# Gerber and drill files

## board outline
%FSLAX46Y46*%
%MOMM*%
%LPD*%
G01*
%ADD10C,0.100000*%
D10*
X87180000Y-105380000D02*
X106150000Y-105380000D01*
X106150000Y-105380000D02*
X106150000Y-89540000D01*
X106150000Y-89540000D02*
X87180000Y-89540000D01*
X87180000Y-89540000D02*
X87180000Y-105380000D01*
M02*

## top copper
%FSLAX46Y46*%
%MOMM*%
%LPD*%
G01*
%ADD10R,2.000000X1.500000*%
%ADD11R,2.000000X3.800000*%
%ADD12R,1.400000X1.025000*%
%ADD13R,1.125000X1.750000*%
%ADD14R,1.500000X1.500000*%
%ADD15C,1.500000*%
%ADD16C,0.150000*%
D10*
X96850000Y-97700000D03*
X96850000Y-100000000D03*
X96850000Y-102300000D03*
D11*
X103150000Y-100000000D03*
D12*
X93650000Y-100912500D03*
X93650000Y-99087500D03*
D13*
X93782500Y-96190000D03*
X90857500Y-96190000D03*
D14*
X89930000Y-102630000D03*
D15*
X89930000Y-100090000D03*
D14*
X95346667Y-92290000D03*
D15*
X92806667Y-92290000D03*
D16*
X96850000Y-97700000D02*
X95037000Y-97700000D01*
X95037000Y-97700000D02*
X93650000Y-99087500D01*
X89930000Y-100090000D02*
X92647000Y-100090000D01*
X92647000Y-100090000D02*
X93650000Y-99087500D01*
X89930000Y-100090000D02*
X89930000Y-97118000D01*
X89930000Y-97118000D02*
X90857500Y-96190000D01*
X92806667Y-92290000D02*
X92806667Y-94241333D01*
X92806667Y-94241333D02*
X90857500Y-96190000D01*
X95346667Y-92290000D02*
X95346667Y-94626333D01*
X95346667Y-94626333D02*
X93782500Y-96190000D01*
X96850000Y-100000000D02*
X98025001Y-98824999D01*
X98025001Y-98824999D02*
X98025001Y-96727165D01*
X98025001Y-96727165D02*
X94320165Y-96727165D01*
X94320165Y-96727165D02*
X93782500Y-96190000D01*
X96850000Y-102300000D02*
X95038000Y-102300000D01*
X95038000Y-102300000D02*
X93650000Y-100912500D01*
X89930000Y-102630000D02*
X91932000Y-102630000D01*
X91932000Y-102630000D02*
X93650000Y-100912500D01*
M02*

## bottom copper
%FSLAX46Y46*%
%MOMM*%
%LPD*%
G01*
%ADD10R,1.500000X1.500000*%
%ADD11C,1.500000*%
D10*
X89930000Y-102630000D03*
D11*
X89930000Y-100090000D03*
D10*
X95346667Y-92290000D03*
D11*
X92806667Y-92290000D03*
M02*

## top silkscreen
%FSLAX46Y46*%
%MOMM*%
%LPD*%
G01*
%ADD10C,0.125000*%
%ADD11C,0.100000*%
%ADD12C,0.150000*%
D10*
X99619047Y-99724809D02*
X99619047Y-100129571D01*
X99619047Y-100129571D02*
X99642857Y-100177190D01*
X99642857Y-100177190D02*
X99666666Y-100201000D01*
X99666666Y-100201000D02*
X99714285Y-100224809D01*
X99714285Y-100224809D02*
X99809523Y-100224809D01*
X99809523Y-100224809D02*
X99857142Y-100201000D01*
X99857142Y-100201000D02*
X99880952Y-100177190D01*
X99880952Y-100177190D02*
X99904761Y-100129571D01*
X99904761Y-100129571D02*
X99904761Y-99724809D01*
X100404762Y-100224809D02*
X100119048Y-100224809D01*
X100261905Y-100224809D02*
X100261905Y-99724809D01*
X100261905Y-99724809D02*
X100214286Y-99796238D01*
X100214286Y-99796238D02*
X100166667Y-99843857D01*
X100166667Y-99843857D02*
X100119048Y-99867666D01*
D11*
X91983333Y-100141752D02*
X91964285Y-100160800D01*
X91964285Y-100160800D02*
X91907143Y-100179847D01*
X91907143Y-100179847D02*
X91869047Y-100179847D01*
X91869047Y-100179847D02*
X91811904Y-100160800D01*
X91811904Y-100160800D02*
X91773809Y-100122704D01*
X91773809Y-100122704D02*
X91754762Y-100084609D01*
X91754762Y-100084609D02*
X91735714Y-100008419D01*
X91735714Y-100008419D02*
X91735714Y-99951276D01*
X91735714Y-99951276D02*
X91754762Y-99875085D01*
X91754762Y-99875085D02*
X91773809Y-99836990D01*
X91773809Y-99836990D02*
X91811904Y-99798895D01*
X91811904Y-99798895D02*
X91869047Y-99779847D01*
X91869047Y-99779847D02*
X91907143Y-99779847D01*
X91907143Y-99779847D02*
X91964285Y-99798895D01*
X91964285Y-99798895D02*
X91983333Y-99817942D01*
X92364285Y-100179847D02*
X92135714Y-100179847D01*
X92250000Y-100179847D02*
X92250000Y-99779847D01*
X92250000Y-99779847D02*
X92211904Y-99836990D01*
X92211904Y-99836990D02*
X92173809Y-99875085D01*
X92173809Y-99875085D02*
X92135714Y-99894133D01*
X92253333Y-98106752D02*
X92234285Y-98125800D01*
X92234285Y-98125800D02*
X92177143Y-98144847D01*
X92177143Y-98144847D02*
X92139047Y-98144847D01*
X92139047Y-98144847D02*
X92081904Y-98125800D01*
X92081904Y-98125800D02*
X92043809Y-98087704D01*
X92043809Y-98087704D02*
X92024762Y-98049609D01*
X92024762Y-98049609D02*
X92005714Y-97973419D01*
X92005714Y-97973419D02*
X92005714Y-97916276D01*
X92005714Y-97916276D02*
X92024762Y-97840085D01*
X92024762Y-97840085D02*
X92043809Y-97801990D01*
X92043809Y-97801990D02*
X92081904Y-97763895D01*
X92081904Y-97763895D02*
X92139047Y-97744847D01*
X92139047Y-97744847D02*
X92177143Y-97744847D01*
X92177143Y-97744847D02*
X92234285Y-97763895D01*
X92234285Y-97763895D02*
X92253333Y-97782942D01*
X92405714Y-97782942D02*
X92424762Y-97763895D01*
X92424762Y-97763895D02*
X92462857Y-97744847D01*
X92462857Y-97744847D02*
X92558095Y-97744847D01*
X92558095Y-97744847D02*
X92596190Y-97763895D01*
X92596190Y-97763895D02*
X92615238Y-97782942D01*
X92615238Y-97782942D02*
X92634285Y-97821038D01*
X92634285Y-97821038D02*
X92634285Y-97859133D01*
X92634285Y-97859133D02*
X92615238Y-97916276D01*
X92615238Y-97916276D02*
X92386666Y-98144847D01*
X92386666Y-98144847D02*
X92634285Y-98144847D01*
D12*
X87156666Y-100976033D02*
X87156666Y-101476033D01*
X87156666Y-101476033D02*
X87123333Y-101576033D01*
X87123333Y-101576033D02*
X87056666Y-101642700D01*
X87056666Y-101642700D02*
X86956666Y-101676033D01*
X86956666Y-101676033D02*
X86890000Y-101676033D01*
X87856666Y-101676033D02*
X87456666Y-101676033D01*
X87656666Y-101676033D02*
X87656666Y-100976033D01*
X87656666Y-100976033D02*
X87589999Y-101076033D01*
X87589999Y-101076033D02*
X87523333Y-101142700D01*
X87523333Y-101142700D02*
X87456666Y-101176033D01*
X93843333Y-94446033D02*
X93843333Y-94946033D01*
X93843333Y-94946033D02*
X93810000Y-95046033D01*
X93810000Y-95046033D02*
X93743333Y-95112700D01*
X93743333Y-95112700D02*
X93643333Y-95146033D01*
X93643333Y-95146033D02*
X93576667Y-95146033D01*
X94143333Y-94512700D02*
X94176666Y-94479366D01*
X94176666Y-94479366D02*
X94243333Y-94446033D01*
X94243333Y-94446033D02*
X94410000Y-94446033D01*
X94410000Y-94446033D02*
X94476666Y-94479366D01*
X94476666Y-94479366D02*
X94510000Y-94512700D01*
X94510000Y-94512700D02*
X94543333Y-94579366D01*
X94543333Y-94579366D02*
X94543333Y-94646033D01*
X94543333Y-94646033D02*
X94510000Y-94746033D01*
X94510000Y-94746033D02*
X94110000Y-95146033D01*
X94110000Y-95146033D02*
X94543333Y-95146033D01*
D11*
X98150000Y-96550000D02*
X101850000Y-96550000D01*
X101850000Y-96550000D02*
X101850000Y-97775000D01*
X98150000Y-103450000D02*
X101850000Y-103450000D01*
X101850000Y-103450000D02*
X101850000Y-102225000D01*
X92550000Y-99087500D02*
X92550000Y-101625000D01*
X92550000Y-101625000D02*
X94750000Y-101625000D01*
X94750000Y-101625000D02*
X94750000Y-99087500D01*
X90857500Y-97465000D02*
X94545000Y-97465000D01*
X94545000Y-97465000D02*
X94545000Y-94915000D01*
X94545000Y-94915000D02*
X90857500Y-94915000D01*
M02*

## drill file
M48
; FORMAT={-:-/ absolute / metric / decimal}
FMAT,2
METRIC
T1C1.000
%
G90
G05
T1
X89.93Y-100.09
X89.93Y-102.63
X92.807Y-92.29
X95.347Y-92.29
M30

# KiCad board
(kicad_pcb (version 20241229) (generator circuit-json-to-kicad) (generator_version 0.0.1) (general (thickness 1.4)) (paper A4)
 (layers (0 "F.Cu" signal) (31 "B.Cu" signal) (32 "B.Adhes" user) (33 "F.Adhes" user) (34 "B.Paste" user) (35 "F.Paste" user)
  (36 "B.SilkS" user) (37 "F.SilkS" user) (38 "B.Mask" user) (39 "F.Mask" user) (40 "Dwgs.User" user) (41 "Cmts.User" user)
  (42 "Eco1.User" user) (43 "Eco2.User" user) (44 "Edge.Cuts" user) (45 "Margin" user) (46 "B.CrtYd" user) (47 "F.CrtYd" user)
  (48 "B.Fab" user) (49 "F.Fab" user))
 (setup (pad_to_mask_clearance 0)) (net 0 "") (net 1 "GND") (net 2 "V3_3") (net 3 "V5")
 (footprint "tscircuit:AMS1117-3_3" (layer F.Cu) (at 100 100 0)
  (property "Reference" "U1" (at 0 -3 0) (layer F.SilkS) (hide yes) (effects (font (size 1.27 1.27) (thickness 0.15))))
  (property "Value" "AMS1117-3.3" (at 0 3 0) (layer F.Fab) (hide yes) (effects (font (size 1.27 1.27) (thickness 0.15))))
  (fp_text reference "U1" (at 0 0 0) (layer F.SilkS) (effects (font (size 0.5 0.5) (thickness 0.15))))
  (fp_line (start -1.85 -3.45) (end 1.85 -3.45) (stroke (width 0.1) (type default)) (layer F.SilkS))
  (fp_line (start 1.85 -3.45) (end 1.85 -2.225) (stroke (width 0.1) (type default)) (layer F.SilkS))
  (fp_line (start -1.85 3.45) (end 1.85 3.45) (stroke (width 0.1) (type default)) (layer F.SilkS))
  (fp_line (start 1.85 3.45) (end 1.85 2.225) (stroke (width 0.1) (type default)) (layer F.SilkS))
  (pad "1" smd rect (at -3.15 -2.3 0) (size 2 1.5) (layers F.Cu F.Paste F.Mask) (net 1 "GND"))
  (pad "2" smd rect (at -3.15 0 0) (size 2 1.5) (layers F.Cu F.Paste F.Mask) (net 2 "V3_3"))
  (pad "3" smd rect (at -3.15 2.3 0) (size 2 1.5) (layers F.Cu F.Paste F.Mask) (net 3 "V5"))
  (pad "4" smd rect (at 3.15 0 0) (size 2 3.8) (layers F.Cu F.Paste F.Mask)))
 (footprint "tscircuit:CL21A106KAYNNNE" (layer F.Cu) (at 93.65 100 90)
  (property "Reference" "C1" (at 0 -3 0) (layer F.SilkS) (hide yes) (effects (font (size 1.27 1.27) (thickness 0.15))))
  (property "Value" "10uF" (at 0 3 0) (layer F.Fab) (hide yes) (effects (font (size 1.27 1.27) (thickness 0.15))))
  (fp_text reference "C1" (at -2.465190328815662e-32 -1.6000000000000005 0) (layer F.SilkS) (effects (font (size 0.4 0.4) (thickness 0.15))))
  (fp_line (start 0.9125 -1.1000000000000005) (end -1.6249999999999998 -1.1000000000000005) (stroke (width 0.1) (type default))
   (layer F.SilkS))
  (fp_line (start -1.6249999999999998 -1.1000000000000005) (end -1.6249999999999998 1.1000000000000005) (stroke (width 0.1) (type default))
   (layer F.SilkS))
  (fp_line (start -1.6249999999999998 1.1000000000000005) (end 0.9125 1.1000000000000005) (stroke (width 0.1) (type default))
   (layer F.SilkS))
  (pad "1" smd rect (at -0.9125 0 0) (size 1.4 1.025) (layers F.Cu F.Paste F.Mask) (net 3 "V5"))
  (pad "2" smd rect (at 0.9125 0 0) (size 1.4 1.025) (layers F.Cu F.Paste F.Mask) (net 1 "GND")))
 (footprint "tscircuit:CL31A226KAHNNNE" (layer F.Cu) (at 92.32 96.19 180)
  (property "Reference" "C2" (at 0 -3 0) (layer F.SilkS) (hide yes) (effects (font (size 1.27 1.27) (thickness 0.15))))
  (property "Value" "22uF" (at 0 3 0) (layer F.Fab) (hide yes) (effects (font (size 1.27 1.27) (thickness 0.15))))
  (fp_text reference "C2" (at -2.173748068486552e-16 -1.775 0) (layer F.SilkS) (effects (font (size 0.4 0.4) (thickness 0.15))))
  (fp_line (start 1.4625000000000001 -1.2749999999999997) (end -2.2249999999999996 -1.2750000000000001) (stroke (width 0.1) (type default))
   (layer F.SilkS))
  (fp_line (start -2.2249999999999996 -1.2750000000000001) (end -2.2249999999999996 1.2749999999999997) (stroke (width 0.1) (type default))
   (layer F.SilkS))
  (fp_line (start -2.2249999999999996 1.2749999999999997) (end 1.4625000000000006 1.2750000000000001) (stroke (width 0.1) (type default))
   (layer F.SilkS))
  (pad "1" smd rect (at -1.4625000000000004 0 0) (size 1.125 1.75) (layers F.Cu F.Paste F.Mask) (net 2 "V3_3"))
  (pad "2" smd rect (at 1.4624999999999995 -4.440892098500626e-16 0) (size 1.125 1.75) (layers F.Cu F.Paste F.Mask) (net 1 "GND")))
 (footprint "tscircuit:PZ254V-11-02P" (layer F.Cu) (at 89.93 101.36 90)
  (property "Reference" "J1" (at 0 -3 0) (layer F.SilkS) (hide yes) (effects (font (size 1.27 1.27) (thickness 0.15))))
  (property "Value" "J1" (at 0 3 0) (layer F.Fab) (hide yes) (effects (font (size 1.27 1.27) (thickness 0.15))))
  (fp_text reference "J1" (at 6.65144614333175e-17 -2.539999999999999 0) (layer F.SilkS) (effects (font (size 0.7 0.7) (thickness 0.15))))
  (pad "1" thru_hole rect (at -1.27 7.776507174585693e-17 0) (size 1.5 1.5) (drill 1) (layers *.Cu *.Mask) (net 3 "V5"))
  (pad "2" thru_hole circle (at 1.27 -7.776507174585693e-17 0) (size 1.5 1.5) (drill 1) (layers *.Cu *.Mask) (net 1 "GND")))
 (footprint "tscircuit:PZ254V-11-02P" (layer F.Cu) (at 94.07666666666667 92.29 180)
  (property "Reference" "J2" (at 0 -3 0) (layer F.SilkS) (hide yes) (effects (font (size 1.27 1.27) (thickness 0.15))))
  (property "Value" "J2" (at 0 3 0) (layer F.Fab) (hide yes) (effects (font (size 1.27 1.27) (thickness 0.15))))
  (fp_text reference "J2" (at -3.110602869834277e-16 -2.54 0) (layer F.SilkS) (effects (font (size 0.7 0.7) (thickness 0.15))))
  (pad "1" thru_hole rect (at -1.2699999999999996 1.555301434917138e-16 0) (size 1.5 1.5) (drill 1) (layers *.Cu *.Mask) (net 2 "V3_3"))
  (pad "2" thru_hole circle (at 1.2699999999999996 -1.555301434917138e-16 0) (size 1.5 1.5) (drill 1) (layers *.Cu *.Mask) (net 1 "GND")))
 (segment (start 96.85 97.7) (end 95.037 97.7) (width 0.15) (layer F.Cu) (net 1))
 (segment (start 95.037 97.7) (end 93.65 99.0875) (width 0.15) (layer F.Cu) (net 1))
 (segment (start 89.93 100.09) (end 92.647 100.09) (width 0.15) (layer F.Cu) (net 1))
 (segment (start 92.647 100.09) (end 93.65 99.0875) (width 0.15) (layer F.Cu) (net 1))
 (segment (start 89.93 100.09) (end 89.93 97.118) (width 0.15) (layer F.Cu) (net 1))
 (segment (start 89.93 97.118) (end 90.8575 96.19) (width 0.15) (layer F.Cu) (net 1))
 (segment (start 92.80666666666667 92.29) (end 92.80666666666667 94.24133333333333) (width 0.15) (layer F.Cu) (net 1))
 (segment (start 92.80666666666667 94.24133333333333) (end 90.8575 96.19) (width 0.15) (layer F.Cu) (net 1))
 (segment (start 95.34666666666666 92.29) (end 95.34666666666666 94.62633333333333) (width 0.15) (layer F.Cu) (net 2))
 (segment (start 95.34666666666666 94.62633333333333) (end 93.7825 96.19) (width 0.15) (layer F.Cu) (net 2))
 (segment (start 96.85 100) (end 98.025001 98.824999) (width 0.15) (layer F.Cu) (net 2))
 (segment (start 98.025001 98.824999) (end 98.025001 96.72716497662654) (width 0.15) (layer F.Cu) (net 2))
 (segment (start 98.025001 96.72716497662654) (end 94.32016497662653 96.72716497662654) (width 0.15) (layer F.Cu) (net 2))
 (segment (start 94.32016497662653 96.72716497662654) (end 93.7825 96.19) (width 0.15) (layer F.Cu) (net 2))
 (segment (start 96.85 102.3) (end 95.038 102.3) (width 0.15) (layer F.Cu) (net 3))
 (segment (start 95.038 102.3) (end 93.65 100.9125) (width 0.15) (layer F.Cu) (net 3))
 (segment (start 89.93 102.63) (end 91.932 102.63) (width 0.15) (layer F.Cu) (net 3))
 (segment (start 91.932 102.63) (end 93.65 100.9125) (width 0.15) (layer F.Cu) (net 3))
 (gr_line (start 87.18 105.38) (end 106.15 105.38) (width 0.1) (layer Edge.Cuts))
 (gr_line (start 106.15 105.38) (end 106.15 89.53999999999999) (width 0.1) (layer Edge.Cuts))
 (gr_line (start 106.15 89.53999999999999) (end 87.18 89.53999999999999) (width 0.1) (layer Edge.Cuts))
 (gr_line (start 87.18 89.53999999999999) (end 87.18 105.38) (width 0.1) (layer Edge.Cuts)))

